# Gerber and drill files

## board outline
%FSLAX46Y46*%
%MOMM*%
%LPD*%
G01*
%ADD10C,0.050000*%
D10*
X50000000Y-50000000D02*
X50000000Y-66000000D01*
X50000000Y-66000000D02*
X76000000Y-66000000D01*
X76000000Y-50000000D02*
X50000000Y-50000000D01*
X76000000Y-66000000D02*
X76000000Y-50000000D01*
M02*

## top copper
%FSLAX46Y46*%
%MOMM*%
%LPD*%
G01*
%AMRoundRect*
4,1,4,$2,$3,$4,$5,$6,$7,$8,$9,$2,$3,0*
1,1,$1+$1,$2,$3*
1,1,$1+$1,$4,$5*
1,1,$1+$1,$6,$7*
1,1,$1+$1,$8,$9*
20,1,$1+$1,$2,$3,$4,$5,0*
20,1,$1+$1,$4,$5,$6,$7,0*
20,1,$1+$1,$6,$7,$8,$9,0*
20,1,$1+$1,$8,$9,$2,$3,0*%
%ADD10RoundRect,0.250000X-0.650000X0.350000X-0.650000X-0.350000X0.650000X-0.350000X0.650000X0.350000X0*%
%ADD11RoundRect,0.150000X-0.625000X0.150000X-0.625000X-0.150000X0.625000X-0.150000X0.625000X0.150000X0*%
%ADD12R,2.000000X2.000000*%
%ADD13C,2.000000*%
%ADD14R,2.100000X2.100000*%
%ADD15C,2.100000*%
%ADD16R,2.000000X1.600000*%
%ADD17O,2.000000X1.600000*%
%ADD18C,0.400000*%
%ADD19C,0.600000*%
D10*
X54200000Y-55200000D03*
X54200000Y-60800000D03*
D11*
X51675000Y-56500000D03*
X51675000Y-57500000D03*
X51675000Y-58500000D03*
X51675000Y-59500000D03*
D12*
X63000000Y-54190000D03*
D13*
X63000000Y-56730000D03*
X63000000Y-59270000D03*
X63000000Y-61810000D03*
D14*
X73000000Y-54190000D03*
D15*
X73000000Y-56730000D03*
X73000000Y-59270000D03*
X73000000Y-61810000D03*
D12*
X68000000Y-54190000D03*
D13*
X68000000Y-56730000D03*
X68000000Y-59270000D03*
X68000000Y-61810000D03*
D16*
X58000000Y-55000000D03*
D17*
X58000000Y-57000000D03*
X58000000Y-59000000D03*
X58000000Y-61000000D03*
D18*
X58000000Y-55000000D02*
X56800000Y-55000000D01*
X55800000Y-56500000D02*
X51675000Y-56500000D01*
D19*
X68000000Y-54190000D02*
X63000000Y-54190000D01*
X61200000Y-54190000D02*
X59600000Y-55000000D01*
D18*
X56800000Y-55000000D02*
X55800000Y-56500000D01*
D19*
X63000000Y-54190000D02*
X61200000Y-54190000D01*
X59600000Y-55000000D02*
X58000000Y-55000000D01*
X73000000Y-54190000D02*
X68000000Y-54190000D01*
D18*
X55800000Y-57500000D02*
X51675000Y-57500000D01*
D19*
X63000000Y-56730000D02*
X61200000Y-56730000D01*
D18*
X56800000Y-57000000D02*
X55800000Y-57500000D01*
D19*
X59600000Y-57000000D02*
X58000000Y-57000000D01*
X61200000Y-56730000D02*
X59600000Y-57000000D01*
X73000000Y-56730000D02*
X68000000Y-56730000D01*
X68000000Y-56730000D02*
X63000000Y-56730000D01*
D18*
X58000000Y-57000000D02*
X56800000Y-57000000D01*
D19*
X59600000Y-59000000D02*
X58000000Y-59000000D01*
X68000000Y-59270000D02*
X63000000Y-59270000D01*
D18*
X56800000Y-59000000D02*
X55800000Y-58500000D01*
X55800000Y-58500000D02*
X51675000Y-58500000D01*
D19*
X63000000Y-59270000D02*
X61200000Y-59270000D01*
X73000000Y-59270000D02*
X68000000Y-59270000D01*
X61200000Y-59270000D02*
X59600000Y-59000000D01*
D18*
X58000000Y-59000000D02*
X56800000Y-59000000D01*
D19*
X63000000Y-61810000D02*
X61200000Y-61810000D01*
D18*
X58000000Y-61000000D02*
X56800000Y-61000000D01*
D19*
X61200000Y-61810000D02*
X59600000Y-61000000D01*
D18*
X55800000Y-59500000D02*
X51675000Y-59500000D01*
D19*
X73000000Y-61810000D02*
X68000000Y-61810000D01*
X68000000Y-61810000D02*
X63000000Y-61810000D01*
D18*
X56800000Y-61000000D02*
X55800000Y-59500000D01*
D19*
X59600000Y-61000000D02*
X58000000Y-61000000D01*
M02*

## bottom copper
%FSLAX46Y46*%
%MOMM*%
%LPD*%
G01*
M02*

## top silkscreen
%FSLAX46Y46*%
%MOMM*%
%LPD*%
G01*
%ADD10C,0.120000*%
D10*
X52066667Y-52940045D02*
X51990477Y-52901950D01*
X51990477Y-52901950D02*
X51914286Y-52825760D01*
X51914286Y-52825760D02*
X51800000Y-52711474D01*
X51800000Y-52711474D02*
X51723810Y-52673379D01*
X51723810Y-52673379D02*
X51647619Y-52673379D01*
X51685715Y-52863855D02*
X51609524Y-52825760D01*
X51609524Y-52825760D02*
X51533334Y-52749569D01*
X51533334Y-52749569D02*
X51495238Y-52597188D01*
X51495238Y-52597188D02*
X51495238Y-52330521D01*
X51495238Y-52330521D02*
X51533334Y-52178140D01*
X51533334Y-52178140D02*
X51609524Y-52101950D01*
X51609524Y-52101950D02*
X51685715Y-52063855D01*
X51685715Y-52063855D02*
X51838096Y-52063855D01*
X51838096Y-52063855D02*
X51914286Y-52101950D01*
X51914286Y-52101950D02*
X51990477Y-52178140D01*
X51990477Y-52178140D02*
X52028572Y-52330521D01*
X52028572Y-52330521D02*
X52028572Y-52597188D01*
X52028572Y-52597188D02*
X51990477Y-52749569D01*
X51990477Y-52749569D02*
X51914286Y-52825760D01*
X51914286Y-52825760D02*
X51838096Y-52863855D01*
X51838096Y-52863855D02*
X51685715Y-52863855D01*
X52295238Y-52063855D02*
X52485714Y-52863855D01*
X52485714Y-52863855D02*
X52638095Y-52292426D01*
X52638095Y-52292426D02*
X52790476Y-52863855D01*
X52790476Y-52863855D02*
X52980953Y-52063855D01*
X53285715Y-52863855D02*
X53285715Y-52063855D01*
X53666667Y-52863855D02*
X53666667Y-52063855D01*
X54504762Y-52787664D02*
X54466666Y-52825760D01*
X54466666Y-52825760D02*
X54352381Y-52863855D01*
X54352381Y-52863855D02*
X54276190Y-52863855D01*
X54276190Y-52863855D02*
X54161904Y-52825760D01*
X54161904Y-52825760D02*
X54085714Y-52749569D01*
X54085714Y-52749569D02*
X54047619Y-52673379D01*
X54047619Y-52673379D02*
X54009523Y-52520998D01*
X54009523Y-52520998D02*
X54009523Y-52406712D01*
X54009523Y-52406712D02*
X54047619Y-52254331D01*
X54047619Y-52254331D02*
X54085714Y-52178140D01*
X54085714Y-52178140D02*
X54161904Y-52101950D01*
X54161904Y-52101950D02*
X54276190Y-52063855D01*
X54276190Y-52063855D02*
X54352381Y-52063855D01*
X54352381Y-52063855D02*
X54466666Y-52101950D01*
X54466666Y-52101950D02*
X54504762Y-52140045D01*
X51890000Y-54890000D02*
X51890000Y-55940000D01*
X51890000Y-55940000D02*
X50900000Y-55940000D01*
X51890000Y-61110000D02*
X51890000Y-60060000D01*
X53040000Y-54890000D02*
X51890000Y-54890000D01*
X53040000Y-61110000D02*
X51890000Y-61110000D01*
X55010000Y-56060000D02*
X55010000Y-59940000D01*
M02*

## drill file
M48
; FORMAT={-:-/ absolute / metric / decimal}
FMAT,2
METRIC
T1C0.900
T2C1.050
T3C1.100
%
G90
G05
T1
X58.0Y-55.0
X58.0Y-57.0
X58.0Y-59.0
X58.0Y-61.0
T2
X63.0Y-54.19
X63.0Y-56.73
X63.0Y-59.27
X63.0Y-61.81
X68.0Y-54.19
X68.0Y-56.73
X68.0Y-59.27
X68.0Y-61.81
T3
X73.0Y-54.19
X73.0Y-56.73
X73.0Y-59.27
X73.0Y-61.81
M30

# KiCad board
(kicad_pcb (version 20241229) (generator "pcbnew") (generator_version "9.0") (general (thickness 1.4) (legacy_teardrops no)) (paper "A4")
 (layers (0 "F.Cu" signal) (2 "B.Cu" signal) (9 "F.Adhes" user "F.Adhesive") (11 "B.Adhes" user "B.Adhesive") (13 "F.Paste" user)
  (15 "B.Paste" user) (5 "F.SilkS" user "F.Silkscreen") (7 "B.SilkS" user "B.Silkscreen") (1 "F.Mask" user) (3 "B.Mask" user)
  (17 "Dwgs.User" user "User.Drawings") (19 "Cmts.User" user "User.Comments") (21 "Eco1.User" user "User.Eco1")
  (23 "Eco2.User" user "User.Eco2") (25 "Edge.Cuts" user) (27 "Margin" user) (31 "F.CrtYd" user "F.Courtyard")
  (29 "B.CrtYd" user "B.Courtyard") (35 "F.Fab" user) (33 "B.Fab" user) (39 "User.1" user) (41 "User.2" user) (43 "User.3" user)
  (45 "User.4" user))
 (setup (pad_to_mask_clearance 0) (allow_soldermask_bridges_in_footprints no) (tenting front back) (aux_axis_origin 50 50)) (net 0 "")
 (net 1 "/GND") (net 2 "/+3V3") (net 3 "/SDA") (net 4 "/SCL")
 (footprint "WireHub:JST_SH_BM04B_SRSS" (layer "F.Cu") (at 53 58 -90)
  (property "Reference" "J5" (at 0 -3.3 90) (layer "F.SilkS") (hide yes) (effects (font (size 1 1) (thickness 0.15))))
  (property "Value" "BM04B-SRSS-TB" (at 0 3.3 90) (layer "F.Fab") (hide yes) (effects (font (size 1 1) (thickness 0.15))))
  (fp_line (start -3.11 1.11) (end -2.06 1.11) (stroke (width 0.12) (type solid)) (layer "F.SilkS"))
  (fp_line (start -2.06 1.11) (end -2.06 2.1) (stroke (width 0.12) (type solid)) (layer "F.SilkS"))
  (fp_line (start 3.11 1.11) (end 2.06 1.11) (stroke (width 0.12) (type solid)) (layer "F.SilkS"))
  (fp_line (start -3.11 -0.04) (end -3.11 1.11) (stroke (width 0.12) (type solid)) (layer "F.SilkS"))
  (fp_line (start 3.11 -0.04) (end 3.11 1.11) (stroke (width 0.12) (type solid)) (layer "F.SilkS"))
  (fp_line (start -1.94 -2.01) (end 1.94 -2.01) (stroke (width 0.12) (type solid)) (layer "F.SilkS"))
  (pad "" smd roundrect (at -2.8 -1.2 270) (size 1.2 1.8) (layers "F.Cu" "F.Mask" "F.Paste") (roundrect_rratio 0.208333))
  (pad "" smd roundrect (at 2.8 -1.2 270) (size 1.2 1.8) (layers "F.Cu" "F.Mask" "F.Paste") (roundrect_rratio 0.208333))
  (pad "1" smd roundrect (at -1.5 1.325 270) (size 0.6 1.55) (layers "F.Cu" "F.Mask" "F.Paste") (roundrect_rratio 0.25) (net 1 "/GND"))
  (pad "2" smd roundrect (at -0.5 1.325 270) (size 0.6 1.55) (layers "F.Cu" "F.Mask" "F.Paste") (roundrect_rratio 0.25) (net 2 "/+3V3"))
  (pad "3" smd roundrect (at 0.5 1.325 270) (size 0.6 1.55) (layers "F.Cu" "F.Mask" "F.Paste") (roundrect_rratio 0.25) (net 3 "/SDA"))
  (pad "4" smd roundrect (at 1.5 1.325 270) (size 0.6 1.55) (layers "F.Cu" "F.Mask" "F.Paste") (roundrect_rratio 0.25) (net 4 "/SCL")))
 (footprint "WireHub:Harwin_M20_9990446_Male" (layer "B.Cu") (at 63 54.19 180)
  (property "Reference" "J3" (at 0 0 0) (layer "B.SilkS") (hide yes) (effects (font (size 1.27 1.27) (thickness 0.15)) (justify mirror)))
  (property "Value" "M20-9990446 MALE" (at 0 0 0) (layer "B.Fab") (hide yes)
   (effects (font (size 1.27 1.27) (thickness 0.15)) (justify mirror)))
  (pad "1" thru_hole rect (at 0 0 180) (size 2 2) (drill 1.05) (layers "*.Cu" "*.Mask") (remove_unused_layers yes) (keep_end_layers no)
   (zone_layer_connections) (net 1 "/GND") (thermal_bridge_angle 45))
  (pad "2" thru_hole circle (at 0 -2.54 180) (size 2 2) (drill 1.05) (layers "*.Cu" "*.Mask") (remove_unused_layers yes)
   (keep_end_layers no) (zone_layer_connections) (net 2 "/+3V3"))
  (pad "3" thru_hole circle (at 0 -5.08 180) (size 2 2) (drill 1.05) (layers "*.Cu" "*.Mask") (remove_unused_layers yes)
   (keep_end_layers no) (zone_layer_connections) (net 3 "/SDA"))
  (pad "4" thru_hole circle (at 0 -7.62 180) (size 2 2) (drill 1.05) (layers "*.Cu" "*.Mask") (remove_unused_layers yes)
   (keep_end_layers no) (zone_layer_connections) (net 4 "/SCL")))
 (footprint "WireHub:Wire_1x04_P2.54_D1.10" (layer "B.Cu") (at 73 54.19 180)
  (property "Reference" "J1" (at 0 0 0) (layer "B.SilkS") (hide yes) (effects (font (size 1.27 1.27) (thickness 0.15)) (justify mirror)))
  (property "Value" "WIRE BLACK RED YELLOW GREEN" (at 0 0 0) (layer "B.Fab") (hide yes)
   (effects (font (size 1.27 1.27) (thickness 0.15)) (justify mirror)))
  (pad "1" thru_hole rect (at 0 0 180) (size 2.1 2.1) (drill 1.1) (layers "*.Cu" "*.Mask") (remove_unused_layers yes) (keep_end_layers no)
   (zone_layer_connections) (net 1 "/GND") (thermal_bridge_angle 45))
  (pad "2" thru_hole circle (at 0 -2.54 180) (size 2.1 2.1) (drill 1.1) (layers "*.Cu" "*.Mask") (remove_unused_layers yes)
   (keep_end_layers no) (zone_layer_connections) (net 2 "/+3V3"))
  (pad "3" thru_hole circle (at 0 -5.08 180) (size 2.1 2.1) (drill 1.1) (layers "*.Cu" "*.Mask") (remove_unused_layers yes)
   (keep_end_layers no) (zone_layer_connections) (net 3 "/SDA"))
  (pad "4" thru_hole circle (at 0 -7.62 180) (size 2.1 2.1) (drill 1.1) (layers "*.Cu" "*.Mask") (remove_unused_layers yes)
   (keep_end_layers no) (zone_layer_connections) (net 4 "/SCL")))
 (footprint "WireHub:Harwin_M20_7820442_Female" (layer "B.Cu") (at 68 54.19 180)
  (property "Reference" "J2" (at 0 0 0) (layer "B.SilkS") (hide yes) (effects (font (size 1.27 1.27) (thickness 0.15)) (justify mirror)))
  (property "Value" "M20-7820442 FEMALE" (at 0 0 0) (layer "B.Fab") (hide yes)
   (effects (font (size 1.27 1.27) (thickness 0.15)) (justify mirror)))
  (pad "1" thru_hole rect (at 0 0 180) (size 2 2) (drill 1.05) (layers "*.Cu" "*.Mask") (remove_unused_layers yes) (keep_end_layers no)
   (zone_layer_connections) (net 1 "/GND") (thermal_bridge_angle 45))
  (pad "2" thru_hole circle (at 0 -2.54 180) (size 2 2) (drill 1.05) (layers "*.Cu" "*.Mask") (remove_unused_layers yes)
   (keep_end_layers no) (zone_layer_connections) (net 2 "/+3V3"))
  (pad "3" thru_hole circle (at 0 -5.08 180) (size 2 2) (drill 1.05) (layers "*.Cu" "*.Mask") (remove_unused_layers yes)
   (keep_end_layers no) (zone_layer_connections) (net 3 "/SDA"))
  (pad "4" thru_hole circle (at 0 -7.62 180) (size 2 2) (drill 1.05) (layers "*.Cu" "*.Mask") (remove_unused_layers yes)
   (keep_end_layers no) (zone_layer_connections) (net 4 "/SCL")))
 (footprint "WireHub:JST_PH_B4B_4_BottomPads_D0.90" (layer "B.Cu") (at 58 55 -90)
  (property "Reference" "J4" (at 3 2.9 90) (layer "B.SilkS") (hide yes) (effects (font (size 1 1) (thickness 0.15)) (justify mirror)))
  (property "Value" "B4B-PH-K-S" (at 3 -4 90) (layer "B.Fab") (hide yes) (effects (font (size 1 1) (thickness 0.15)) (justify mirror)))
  (pad "1" thru_hole rect (at 0 0 270) (size 1.6 2) (drill 0.9) (layers "*.Cu" "*.Mask") (remove_unused_layers yes) (keep_end_layers no)
   (zone_layer_connections) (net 1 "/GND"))
  (pad "2" thru_hole oval (at 2 0 270) (size 1.6 2) (drill 0.9) (layers "*.Cu" "*.Mask") (remove_unused_layers yes) (keep_end_layers no)
   (zone_layer_connections) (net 2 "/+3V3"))
  (pad "3" thru_hole oval (at 4 0 270) (size 1.6 2) (drill 0.9) (layers "*.Cu" "*.Mask") (remove_unused_layers yes) (keep_end_layers no)
   (zone_layer_connections) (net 3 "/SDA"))
  (pad "4" thru_hole oval (at 6 0 270) (size 1.6 2) (drill 0.9) (layers "*.Cu" "*.Mask") (remove_unused_layers yes) (keep_end_layers no)
   (zone_layer_connections) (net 4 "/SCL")))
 (gr_line (start 50 50) (end 50 66) (stroke (width 0.05) (type default)) (layer "Edge.Cuts"))
 (gr_line (start 50 66) (end 76 66) (stroke (width 0.05) (type default)) (layer "Edge.Cuts"))
 (gr_line (start 76 50) (end 50 50) (stroke (width 0.05) (type default)) (layer "Edge.Cuts"))
 (gr_line (start 76 66) (end 76 50) (stroke (width 0.05) (type default)) (layer "Edge.Cuts"))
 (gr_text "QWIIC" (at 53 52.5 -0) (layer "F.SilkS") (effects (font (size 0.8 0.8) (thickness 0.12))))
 (segment (start 58 55) (end 56.8 55) (width 0.4) (layer "F.Cu") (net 1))
 (segment (start 55.8 56.5) (end 51.675 56.5) (width 0.4) (layer "F.Cu") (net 1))
 (segment (start 68 54.19) (end 63 54.19) (width 0.6) (layer "F.Cu") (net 1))
 (segment (start 61.2 54.19) (end 59.6 55) (width 0.6) (layer "F.Cu") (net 1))
 (segment (start 56.8 55) (end 55.8 56.5) (width 0.4) (layer "F.Cu") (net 1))
 (segment (start 63 54.19) (end 61.2 54.19) (width 0.6) (layer "F.Cu") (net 1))
 (segment (start 59.6 55) (end 58 55) (width 0.6) (layer "F.Cu") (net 1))
 (segment (start 73 54.19) (end 68 54.19) (width 0.6) (layer "F.Cu") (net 1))
 (segment (start 55.8 57.5) (end 51.675 57.5) (width 0.4) (layer "F.Cu") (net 2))
 (segment (start 63 56.73) (end 61.2 56.73) (width 0.6) (layer "F.Cu") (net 2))
 (segment (start 56.8 57) (end 55.8 57.5) (width 0.4) (layer "F.Cu") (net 2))
 (segment (start 59.6 57) (end 58 57) (width 0.6) (layer "F.Cu") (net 2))
 (segment (start 61.2 56.73) (end 59.6 57) (width 0.6) (layer "F.Cu") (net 2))
 (segment (start 73 56.73) (end 68 56.73) (width 0.6) (layer "F.Cu") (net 2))
 (segment (start 68 56.73) (end 63 56.73) (width 0.6) (layer "F.Cu") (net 2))
 (segment (start 58 57) (end 56.8 57) (width 0.4) (layer "F.Cu") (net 2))
 (segment (start 59.6 59) (end 58 59) (width 0.6) (layer "F.Cu") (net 3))
 (segment (start 68 59.27) (end 63 59.27) (width 0.6) (layer "F.Cu") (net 3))
 (segment (start 56.8 59) (end 55.8 58.5) (width 0.4) (layer "F.Cu") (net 3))
 (segment (start 55.8 58.5) (end 51.675 58.5) (width 0.4) (layer "F.Cu") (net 3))
 (segment (start 63 59.27) (end 61.2 59.27) (width 0.6) (layer "F.Cu") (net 3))
 (segment (start 73 59.27) (end 68 59.27) (width 0.6) (layer "F.Cu") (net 3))
 (segment (start 61.2 59.27) (end 59.6 59) (width 0.6) (layer "F.Cu") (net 3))
 (segment (start 58 59) (end 56.8 59) (width 0.4) (layer "F.Cu") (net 3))
 (segment (start 63 61.81) (end 61.2 61.81) (width 0.6) (layer "F.Cu") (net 4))
 (segment (start 58 61) (end 56.8 61) (width 0.4) (layer "F.Cu") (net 4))
 (segment (start 61.2 61.81) (end 59.6 61) (width 0.6) (layer "F.Cu") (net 4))
 (segment (start 55.8 59.5) (end 51.675 59.5) (width 0.4) (layer "F.Cu") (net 4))
 (segment (start 73 61.81) (end 68 61.81) (width 0.6) (layer "F.Cu") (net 4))
 (segment (start 68 61.81) (end 63 61.81) (width 0.6) (layer "F.Cu") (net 4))
 (segment (start 56.8 61) (end 55.8 59.5) (width 0.4) (layer "F.Cu") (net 4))
 (segment (start 59.6 61) (end 58 61) (width 0.6) (layer "F.Cu") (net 4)))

